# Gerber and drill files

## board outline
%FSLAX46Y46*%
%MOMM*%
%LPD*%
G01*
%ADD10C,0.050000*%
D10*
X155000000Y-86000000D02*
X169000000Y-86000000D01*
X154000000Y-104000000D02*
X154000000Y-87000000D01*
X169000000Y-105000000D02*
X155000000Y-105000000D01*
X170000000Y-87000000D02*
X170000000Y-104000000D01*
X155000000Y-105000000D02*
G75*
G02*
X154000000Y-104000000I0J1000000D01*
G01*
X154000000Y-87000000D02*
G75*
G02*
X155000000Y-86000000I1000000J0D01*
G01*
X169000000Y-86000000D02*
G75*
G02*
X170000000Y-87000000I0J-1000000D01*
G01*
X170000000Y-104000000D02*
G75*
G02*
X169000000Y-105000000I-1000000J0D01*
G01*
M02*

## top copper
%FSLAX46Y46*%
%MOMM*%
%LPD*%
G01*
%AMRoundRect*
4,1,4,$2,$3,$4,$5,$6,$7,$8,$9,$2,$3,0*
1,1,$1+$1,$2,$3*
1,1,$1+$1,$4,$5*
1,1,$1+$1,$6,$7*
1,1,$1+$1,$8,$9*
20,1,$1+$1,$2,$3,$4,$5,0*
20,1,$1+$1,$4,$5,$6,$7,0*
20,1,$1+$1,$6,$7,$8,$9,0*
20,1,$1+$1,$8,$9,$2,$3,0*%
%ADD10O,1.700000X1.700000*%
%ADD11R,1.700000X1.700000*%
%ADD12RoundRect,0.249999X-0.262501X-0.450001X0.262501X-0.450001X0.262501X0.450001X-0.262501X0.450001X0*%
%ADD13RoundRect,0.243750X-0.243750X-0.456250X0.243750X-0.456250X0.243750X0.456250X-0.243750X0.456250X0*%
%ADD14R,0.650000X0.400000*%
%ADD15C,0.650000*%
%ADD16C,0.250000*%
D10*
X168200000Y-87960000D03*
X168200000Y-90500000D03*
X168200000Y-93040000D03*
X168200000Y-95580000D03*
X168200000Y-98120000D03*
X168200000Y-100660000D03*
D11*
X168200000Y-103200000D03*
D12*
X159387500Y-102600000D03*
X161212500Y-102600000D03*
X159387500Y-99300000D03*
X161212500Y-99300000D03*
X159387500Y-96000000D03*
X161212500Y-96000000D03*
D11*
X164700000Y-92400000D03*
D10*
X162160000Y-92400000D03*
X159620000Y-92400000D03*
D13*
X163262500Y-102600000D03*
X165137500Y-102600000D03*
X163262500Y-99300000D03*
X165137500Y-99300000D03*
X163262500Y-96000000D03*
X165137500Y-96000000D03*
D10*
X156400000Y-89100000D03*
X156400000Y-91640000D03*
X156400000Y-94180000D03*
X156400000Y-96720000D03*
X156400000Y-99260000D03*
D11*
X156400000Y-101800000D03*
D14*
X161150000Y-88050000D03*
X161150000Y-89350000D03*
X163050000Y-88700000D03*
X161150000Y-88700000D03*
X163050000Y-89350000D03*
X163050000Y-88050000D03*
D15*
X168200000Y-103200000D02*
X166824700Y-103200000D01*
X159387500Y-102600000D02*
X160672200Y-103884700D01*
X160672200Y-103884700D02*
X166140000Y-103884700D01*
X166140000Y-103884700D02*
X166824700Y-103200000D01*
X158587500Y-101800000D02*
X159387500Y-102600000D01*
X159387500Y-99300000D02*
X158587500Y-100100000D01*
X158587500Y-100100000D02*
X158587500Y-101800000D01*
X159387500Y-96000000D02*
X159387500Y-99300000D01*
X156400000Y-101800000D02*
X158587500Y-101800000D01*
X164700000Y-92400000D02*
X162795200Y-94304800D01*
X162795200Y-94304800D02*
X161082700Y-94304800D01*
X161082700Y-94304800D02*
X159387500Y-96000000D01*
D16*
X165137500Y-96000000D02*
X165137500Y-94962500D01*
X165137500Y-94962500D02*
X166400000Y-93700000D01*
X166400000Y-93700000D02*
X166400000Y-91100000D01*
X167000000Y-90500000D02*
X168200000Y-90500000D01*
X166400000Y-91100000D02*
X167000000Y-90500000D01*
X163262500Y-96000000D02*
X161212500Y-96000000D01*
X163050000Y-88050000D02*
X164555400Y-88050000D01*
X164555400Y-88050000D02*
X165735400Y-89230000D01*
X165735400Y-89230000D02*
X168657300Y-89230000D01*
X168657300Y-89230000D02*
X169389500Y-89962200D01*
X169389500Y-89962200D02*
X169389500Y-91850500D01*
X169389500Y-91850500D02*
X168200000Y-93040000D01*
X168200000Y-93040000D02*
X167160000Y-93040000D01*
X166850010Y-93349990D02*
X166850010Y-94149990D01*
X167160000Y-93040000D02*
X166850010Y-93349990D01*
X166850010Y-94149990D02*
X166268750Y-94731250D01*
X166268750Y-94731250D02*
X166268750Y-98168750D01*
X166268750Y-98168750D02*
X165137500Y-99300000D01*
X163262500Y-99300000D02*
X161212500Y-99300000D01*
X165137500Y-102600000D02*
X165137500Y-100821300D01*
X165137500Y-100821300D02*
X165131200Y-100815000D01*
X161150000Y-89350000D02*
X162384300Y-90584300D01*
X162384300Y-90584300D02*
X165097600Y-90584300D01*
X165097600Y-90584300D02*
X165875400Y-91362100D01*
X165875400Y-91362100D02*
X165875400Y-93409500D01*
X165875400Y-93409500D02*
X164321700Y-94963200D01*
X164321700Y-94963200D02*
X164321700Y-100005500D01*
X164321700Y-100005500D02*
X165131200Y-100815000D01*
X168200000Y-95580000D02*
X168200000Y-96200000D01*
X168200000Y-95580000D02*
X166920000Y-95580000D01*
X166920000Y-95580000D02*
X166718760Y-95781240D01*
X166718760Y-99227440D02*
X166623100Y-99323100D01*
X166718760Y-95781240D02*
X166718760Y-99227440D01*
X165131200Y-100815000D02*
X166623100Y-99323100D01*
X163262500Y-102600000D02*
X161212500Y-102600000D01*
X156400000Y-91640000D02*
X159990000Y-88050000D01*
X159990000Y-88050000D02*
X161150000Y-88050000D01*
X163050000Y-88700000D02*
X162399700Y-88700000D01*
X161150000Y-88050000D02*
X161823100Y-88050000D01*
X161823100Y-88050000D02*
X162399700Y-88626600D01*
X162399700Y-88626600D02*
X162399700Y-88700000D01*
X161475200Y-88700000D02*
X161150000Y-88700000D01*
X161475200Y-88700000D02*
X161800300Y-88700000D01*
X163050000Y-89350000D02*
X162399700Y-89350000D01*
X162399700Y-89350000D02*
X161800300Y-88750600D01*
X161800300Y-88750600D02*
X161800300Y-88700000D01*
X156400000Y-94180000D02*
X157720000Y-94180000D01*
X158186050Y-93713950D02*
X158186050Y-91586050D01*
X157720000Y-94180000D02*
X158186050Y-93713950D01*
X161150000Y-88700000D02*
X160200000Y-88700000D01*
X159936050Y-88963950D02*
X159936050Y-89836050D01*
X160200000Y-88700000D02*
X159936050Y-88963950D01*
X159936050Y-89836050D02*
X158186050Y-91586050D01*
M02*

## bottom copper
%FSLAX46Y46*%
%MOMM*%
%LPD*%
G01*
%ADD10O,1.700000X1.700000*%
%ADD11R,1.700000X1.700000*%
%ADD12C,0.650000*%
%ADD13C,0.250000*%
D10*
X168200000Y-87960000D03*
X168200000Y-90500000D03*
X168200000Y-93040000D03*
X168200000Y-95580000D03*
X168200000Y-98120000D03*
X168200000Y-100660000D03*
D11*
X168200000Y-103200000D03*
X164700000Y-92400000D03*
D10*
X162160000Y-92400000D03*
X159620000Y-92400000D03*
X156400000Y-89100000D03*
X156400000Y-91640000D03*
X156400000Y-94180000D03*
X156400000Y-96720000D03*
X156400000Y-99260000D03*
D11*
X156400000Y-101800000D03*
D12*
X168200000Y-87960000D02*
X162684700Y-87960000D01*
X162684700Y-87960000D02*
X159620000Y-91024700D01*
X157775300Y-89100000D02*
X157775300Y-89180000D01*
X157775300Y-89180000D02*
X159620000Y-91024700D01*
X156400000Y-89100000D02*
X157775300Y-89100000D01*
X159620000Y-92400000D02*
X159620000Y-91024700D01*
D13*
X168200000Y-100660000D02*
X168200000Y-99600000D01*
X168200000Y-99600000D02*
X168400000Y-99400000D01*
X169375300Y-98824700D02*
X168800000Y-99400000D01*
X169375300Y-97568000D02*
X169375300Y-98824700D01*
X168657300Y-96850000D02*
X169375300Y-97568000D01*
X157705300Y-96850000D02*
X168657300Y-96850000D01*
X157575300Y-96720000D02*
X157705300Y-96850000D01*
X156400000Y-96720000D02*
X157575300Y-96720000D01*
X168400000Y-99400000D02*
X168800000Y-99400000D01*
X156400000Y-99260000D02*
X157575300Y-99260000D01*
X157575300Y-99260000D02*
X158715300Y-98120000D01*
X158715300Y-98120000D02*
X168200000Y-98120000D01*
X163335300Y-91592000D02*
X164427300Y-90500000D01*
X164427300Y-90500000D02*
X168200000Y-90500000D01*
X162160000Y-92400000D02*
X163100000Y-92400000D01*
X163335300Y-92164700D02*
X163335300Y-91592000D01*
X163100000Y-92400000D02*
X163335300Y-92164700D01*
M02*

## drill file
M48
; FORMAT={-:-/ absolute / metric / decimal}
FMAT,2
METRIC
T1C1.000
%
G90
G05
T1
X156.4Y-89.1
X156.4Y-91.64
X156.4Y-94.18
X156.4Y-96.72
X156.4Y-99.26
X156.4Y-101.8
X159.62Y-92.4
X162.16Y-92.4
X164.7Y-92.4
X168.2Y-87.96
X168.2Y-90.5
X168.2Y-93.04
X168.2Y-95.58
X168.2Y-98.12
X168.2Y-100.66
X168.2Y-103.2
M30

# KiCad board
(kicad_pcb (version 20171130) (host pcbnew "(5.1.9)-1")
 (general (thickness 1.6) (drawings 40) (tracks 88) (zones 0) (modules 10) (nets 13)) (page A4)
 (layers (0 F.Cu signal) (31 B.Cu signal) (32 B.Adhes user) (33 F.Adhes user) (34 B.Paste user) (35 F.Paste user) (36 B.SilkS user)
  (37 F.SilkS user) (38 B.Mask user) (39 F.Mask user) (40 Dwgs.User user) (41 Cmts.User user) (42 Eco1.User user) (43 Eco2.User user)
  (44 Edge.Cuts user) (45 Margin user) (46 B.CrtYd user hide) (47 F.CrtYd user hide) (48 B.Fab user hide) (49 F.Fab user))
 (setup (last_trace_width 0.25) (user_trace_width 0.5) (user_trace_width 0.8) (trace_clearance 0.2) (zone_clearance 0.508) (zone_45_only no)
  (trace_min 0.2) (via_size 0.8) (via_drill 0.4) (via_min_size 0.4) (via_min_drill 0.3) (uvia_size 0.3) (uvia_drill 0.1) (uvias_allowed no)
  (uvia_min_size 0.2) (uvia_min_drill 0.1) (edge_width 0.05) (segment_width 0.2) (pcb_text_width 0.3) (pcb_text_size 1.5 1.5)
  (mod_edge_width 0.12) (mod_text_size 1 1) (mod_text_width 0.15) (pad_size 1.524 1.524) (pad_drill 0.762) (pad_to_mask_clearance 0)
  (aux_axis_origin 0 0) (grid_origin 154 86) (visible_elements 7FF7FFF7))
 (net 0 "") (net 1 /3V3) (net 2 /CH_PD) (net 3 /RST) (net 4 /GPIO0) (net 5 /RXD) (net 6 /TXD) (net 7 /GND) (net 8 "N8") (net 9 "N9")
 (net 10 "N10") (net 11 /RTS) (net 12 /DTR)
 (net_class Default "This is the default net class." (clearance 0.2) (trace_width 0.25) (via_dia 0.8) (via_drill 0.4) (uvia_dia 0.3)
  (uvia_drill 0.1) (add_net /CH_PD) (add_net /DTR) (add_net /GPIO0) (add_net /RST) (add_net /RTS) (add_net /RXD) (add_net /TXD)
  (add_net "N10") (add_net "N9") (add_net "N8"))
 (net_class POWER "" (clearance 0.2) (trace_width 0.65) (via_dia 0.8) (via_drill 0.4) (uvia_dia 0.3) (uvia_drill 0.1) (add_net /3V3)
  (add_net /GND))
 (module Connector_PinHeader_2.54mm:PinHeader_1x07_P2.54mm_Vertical (layer F.Cu) (at 168.2 103.2 180)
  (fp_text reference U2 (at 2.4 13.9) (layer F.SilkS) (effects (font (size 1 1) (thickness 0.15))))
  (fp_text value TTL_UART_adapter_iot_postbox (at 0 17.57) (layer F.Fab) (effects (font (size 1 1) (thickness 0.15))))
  (pad 7 thru_hole oval (at 0 15.24 180) (size 1.7 1.7) (drill 1) (layers *.Cu *.Mask) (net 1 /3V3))
  (pad 6 thru_hole oval (at 0 12.7 180) (size 1.7 1.7) (drill 1) (layers *.Cu *.Mask) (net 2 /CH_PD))
  (pad 5 thru_hole oval (at 0 10.16 180) (size 1.7 1.7) (drill 1) (layers *.Cu *.Mask) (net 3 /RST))
  (pad 4 thru_hole oval (at 0 7.62 180) (size 1.7 1.7) (drill 1) (layers *.Cu *.Mask) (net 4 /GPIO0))
  (pad 3 thru_hole oval (at 0 5.08 180) (size 1.7 1.7) (drill 1) (layers *.Cu *.Mask) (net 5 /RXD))
  (pad 2 thru_hole oval (at 0 2.54 180) (size 1.7 1.7) (drill 1) (layers *.Cu *.Mask) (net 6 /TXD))
  (pad 1 thru_hole rect (at 0 0 180) (size 1.7 1.7) (drill 1) (layers *.Cu *.Mask) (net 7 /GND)))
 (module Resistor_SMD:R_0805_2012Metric (layer F.Cu) (at 160.3 102.6)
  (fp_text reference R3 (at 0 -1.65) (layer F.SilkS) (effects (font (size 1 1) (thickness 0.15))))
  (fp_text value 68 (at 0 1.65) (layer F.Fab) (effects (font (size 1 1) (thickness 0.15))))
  (pad 1 smd roundrect (at -0.9125 0) (size 1.025 1.4) (layers F.Cu F.Paste F.Mask) (roundrect_rratio 0.2439014634146341) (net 7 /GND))
  (pad 2 smd roundrect (at 0.9125 0) (size 1.025 1.4) (layers F.Cu F.Paste F.Mask) (roundrect_rratio 0.2439014634146341) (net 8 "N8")))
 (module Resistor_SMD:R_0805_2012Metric (layer F.Cu) (at 160.3 99.3)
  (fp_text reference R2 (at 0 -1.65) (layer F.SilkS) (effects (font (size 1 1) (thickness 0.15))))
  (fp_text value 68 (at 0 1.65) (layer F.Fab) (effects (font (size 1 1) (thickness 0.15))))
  (pad 1 smd roundrect (at -0.9125 0) (size 1.025 1.4) (layers F.Cu F.Paste F.Mask) (roundrect_rratio 0.2439014634146341) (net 7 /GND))
  (pad 2 smd roundrect (at 0.9125 0) (size 1.025 1.4) (layers F.Cu F.Paste F.Mask) (roundrect_rratio 0.2439014634146341) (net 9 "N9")))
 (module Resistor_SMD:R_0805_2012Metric (layer F.Cu) (at 160.3 96)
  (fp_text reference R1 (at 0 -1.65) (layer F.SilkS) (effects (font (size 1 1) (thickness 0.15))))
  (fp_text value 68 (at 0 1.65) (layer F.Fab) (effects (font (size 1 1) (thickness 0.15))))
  (pad 1 smd roundrect (at -0.9125 0) (size 1.025 1.4) (layers F.Cu F.Paste F.Mask) (roundrect_rratio 0.2439014634146341) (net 7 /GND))
  (pad 2 smd roundrect (at 0.9125 0) (size 1.025 1.4) (layers F.Cu F.Paste F.Mask) (roundrect_rratio 0.2439014634146341) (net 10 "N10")))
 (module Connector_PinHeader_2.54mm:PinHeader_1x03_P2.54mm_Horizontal (layer B.Cu) (at 164.7 92.4 90)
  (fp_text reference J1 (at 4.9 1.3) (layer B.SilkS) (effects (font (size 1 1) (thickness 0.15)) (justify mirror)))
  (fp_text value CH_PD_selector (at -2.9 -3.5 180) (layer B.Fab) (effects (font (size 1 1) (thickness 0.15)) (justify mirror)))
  (pad 1 thru_hole rect (at 0 0 90) (size 1.7 1.7) (drill 1) (layers *.Cu *.Mask) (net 7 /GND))
  (pad 2 thru_hole oval (at 0 -2.54 90) (size 1.7 1.7) (drill 1) (layers *.Cu *.Mask) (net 2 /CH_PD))
  (pad 3 thru_hole oval (at 0 -5.08 90) (size 1.7 1.7) (drill 1) (layers *.Cu *.Mask) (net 1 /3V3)))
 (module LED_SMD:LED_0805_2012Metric (layer F.Cu) (at 164.2 102.6)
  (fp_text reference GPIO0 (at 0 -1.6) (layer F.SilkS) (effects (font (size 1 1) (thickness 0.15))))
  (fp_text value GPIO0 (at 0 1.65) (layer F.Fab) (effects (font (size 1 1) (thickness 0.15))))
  (pad 1 smd roundrect (at -0.9375 0) (size 0.975 1.4) (layers F.Cu F.Paste F.Mask) (roundrect_rratio 0.25) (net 8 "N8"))
  (pad 2 smd roundrect (at 0.9375 0) (size 0.975 1.4) (layers F.Cu F.Paste F.Mask) (roundrect_rratio 0.25) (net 4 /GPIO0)))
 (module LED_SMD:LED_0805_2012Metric (layer F.Cu) (at 164.2 99.3)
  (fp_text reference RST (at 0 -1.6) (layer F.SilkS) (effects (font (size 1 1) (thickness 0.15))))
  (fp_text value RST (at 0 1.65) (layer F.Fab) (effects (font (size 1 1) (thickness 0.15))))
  (pad 1 smd roundrect (at -0.9375 0) (size 0.975 1.4) (layers F.Cu F.Paste F.Mask) (roundrect_rratio 0.25) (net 9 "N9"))
  (pad 2 smd roundrect (at 0.9375 0) (size 0.975 1.4) (layers F.Cu F.Paste F.Mask) (roundrect_rratio 0.25) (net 3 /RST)))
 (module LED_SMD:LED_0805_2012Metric (layer F.Cu) (at 164.2 96)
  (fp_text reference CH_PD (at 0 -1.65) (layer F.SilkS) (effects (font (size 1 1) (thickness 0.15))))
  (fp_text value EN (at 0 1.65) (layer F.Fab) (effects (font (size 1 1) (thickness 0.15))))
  (pad 1 smd roundrect (at -0.9375 0) (size 0.975 1.4) (layers F.Cu F.Paste F.Mask) (roundrect_rratio 0.25) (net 10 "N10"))
  (pad 2 smd roundrect (at 0.9375 0) (size 0.975 1.4) (layers F.Cu F.Paste F.Mask) (roundrect_rratio 0.25) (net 2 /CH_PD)))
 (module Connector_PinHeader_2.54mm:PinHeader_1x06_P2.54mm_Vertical (layer F.Cu) (at 156.4 101.8 180)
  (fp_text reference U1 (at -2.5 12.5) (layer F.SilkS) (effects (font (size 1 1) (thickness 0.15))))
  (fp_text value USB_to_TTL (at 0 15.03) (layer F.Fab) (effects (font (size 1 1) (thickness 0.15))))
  (pad 6 thru_hole oval (at 0 12.7 180) (size 1.7 1.7) (drill 1) (layers *.Cu *.Mask) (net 1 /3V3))
  (pad 5 thru_hole oval (at 0 10.16 180) (size 1.7 1.7) (drill 1) (layers *.Cu *.Mask) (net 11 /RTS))
  (pad 4 thru_hole oval (at 0 7.62 180) (size 1.7 1.7) (drill 1) (layers *.Cu *.Mask) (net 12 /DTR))
  (pad 3 thru_hole oval (at 0 5.08 180) (size 1.7 1.7) (drill 1) (layers *.Cu *.Mask) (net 6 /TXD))
  (pad 2 thru_hole oval (at 0 2.54 180) (size 1.7 1.7) (drill 1) (layers *.Cu *.Mask) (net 5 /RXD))
  (pad 1 thru_hole rect (at 0 0 180) (size 1.7 1.7) (drill 1) (layers *.Cu *.Mask) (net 7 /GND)))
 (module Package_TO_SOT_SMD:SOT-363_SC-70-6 (layer F.Cu) (at 162.1 88.7)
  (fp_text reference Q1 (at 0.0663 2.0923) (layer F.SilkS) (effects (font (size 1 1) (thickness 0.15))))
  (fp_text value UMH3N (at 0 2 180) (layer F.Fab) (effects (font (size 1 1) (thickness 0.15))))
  (pad 1 smd rect (at -0.95 -0.65) (size 0.65 0.4) (layers F.Cu F.Paste F.Mask) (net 11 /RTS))
  (pad 3 smd rect (at -0.95 0.65) (size 0.65 0.4) (layers F.Cu F.Paste F.Mask) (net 4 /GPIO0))
  (pad 5 smd rect (at 0.95 0) (size 0.65 0.4) (layers F.Cu F.Paste F.Mask) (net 11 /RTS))
  (pad 2 smd rect (at -0.95 0) (size 0.65 0.4) (layers F.Cu F.Paste F.Mask) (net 12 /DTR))
  (pad 4 smd rect (at 0.95 0.65) (size 0.65 0.4) (layers F.Cu F.Paste F.Mask) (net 12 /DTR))
  (pad 6 smd rect (at 0.95 -0.65) (size 0.65 0.4) (layers F.Cu F.Paste F.Mask) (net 3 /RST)))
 (gr_line (start 155 86) (end 169 86) (layer Edge.Cuts) (width 0.05))
 (gr_line (start 154 104) (end 154 87) (layer Edge.Cuts) (width 0.05))
 (gr_line (start 169 105) (end 155 105) (layer Edge.Cuts) (width 0.05))
 (gr_line (start 170 87) (end 170 104) (layer Edge.Cuts) (width 0.05))
 (gr_arc (start 155 104) (end 154 104) (angle -90) (layer Edge.Cuts) (width 0.05))
 (gr_arc (start 155 87) (end 155 86) (angle -90) (layer Edge.Cuts) (width 0.05))
 (gr_arc (start 169 87) (end 170 87) (angle -90) (layer Edge.Cuts) (width 0.05))
 (gr_arc (start 169 104) (end 169 105) (angle -90) (layer Edge.Cuts) (width 0.05))
 (segment (start 168.2 87.96) (end 162.6847 87.96) (width 0.65) (layer B.Cu) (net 1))
 (segment (start 162.6847 87.96) (end 159.62 91.0247) (width 0.65) (layer B.Cu) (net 1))
 (segment (start 157.7753 89.1) (end 157.7753 89.18) (width 0.65) (layer B.Cu) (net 1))
 (segment (start 157.7753 89.18) (end 159.62 91.0247) (width 0.65) (layer B.Cu) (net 1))
 (segment (start 156.4 89.1) (end 157.7753 89.1) (width 0.65) (layer B.Cu) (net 1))
 (segment (start 159.62 92.4) (end 159.62 91.0247) (width 0.65) (layer B.Cu) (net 1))
 (segment (start 168.2 100.66) (end 168.2 99.6) (width 0.25) (layer B.Cu) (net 6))
 (segment (start 168.2 99.6) (end 168.4 99.4) (width 0.25) (layer B.Cu) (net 6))
 (segment (start 169.3753 98.8247) (end 168.8 99.4) (width 0.25) (layer B.Cu) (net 6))
 (segment (start 169.3753 97.568) (end 169.3753 98.8247) (width 0.25) (layer B.Cu) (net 6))
 (segment (start 168.6573 96.85) (end 169.3753 97.568) (width 0.25) (layer B.Cu) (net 6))
 (segment (start 157.7053 96.85) (end 168.6573 96.85) (width 0.25) (layer B.Cu) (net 6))
 (segment (start 157.5753 96.72) (end 157.7053 96.85) (width 0.25) (layer B.Cu) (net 6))
 (segment (start 156.4 96.72) (end 157.5753 96.72) (width 0.25) (layer B.Cu) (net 6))
 (segment (start 168.4 99.4) (end 168.8 99.4) (width 0.25) (layer B.Cu) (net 6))
 (segment (start 156.4 99.26) (end 157.5753 99.26) (width 0.25) (layer B.Cu) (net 5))
 (segment (start 157.5753 99.26) (end 158.7153 98.12) (width 0.25) (layer B.Cu) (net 5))
 (segment (start 158.7153 98.12) (end 168.2 98.12) (width 0.25) (layer B.Cu) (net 5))
 (segment (start 168.2 103.2) (end 166.8247 103.2) (width 0.65) (layer F.Cu) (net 7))
 (segment (start 159.3875 102.6) (end 160.6722 103.8847) (width 0.65) (layer F.Cu) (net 7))
 (segment (start 160.6722 103.8847) (end 166.14 103.8847) (width 0.65) (layer F.Cu) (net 7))
 (segment (start 166.14 103.8847) (end 166.8247 103.2) (width 0.65) (layer F.Cu) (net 7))
 (segment (start 158.5875 101.8) (end 159.3875 102.6) (width 0.65) (layer F.Cu) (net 7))
 (segment (start 159.3875 99.3) (end 158.5875 100.1) (width 0.65) (layer F.Cu) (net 7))
 (segment (start 158.5875 100.1) (end 158.5875 101.8) (width 0.65) (layer F.Cu) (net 7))
 (segment (start 159.3875 96) (end 159.3875 99.3) (width 0.65) (layer F.Cu) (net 7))
 (segment (start 156.4 101.8) (end 158.5875 101.8) (width 0.65) (layer F.Cu) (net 7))
 (segment (start 164.7 92.4) (end 162.7952 94.3048) (width 0.65) (layer F.Cu) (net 7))
 (segment (start 162.7952 94.3048) (end 161.0827 94.3048) (width 0.65) (layer F.Cu) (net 7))
 (segment (start 161.0827 94.3048) (end 159.3875 96) (width 0.65) (layer F.Cu) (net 7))
 (segment (start 163.3353 91.592) (end 164.4273 90.5) (width 0.25) (layer B.Cu) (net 2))
 (segment (start 164.4273 90.5) (end 168.2 90.5) (width 0.25) (layer B.Cu) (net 2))
 (segment (start 165.1375 96) (end 165.1375 94.9625) (width 0.25) (layer F.Cu) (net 2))
 (segment (start 165.1375 94.9625) (end 166.4 93.7) (width 0.25) (layer F.Cu) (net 2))
 (segment (start 166.4 93.7) (end 166.4 91.1) (width 0.25) (layer F.Cu) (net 2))
 (segment (start 167 90.5) (end 168.2 90.5) (width 0.25) (layer F.Cu) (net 2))
 (segment (start 166.4 91.1) (end 167 90.5) (width 0.25) (layer F.Cu) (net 2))
 (segment (start 162.16 92.4) (end 163.1 92.4) (width 0.25) (layer B.Cu) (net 2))
 (segment (start 163.3353 92.1647) (end 163.3353 91.592) (width 0.25) (layer B.Cu) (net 2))
 (segment (start 163.1 92.4) (end 163.3353 92.1647) (width 0.25) (layer B.Cu) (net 2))
 (segment (start 163.2625 96) (end 161.2125 96) (width 0.25) (layer F.Cu) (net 10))
 (segment (start 163.05 88.05) (end 164.5554 88.05) (width 0.25) (layer F.Cu) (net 3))
 (segment (start 164.5554 88.05) (end 165.7354 89.23) (width 0.25) (layer F.Cu) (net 3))
 (segment (start 165.7354 89.23) (end 168.6573 89.23) (width 0.25) (layer F.Cu) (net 3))
 (segment (start 168.6573 89.23) (end 169.3895 89.9622) (width 0.25) (layer F.Cu) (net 3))
 (segment (start 169.3895 89.9622) (end 169.3895 91.8505) (width 0.25) (layer F.Cu) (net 3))
 (segment (start 169.3895 91.8505) (end 168.2 93.04) (width 0.25) (layer F.Cu) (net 3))
 (segment (start 168.2 93.04) (end 167.16 93.04) (width 0.25) (layer F.Cu) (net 3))
 (segment (start 166.85001 93.34999) (end 166.85001 94.14999) (width 0.25) (layer F.Cu) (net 3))
 (segment (start 167.16 93.04) (end 166.85001 93.34999) (width 0.25) (layer F.Cu) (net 3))
 (segment (start 166.85001 94.14999) (end 166.26875 94.73125) (width 0.25) (layer F.Cu) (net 3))
 (segment (start 166.26875 94.73125) (end 166.26875 98.16875) (width 0.25) (layer F.Cu) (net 3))
 (segment (start 166.26875 98.16875) (end 165.1375 99.3) (width 0.25) (layer F.Cu) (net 3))
 (segment (start 163.2625 99.3) (end 161.2125 99.3) (width 0.25) (layer F.Cu) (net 9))
 (segment (start 165.1375 102.6) (end 165.1375 100.8213) (width 0.25) (layer F.Cu) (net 4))
 (segment (start 165.1375 100.8213) (end 165.1312 100.815) (width 0.25) (layer F.Cu) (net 4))
 (segment (start 161.15 89.35) (end 162.3843 90.5843) (width 0.25) (layer F.Cu) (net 4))
 (segment (start 162.3843 90.5843) (end 165.0976 90.5843) (width 0.25) (layer F.Cu) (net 4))
 (segment (start 165.0976 90.5843) (end 165.8754 91.3621) (width 0.25) (layer F.Cu) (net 4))
 (segment (start 165.8754 91.3621) (end 165.8754 93.4095) (width 0.25) (layer F.Cu) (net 4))
 (segment (start 165.8754 93.4095) (end 164.3217 94.9632) (width 0.25) (layer F.Cu) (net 4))
 (segment (start 164.3217 94.9632) (end 164.3217 100.0055) (width 0.25) (layer F.Cu) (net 4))
 (segment (start 164.3217 100.0055) (end 165.1312 100.815) (width 0.25) (layer F.Cu) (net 4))
 (segment (start 168.2 95.58) (end 168.2 96.2) (width 0.25) (layer F.Cu) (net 4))
 (segment (start 168.2 95.58) (end 166.92 95.58) (width 0.25) (layer F.Cu) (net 4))
 (segment (start 166.92 95.58) (end 166.71876 95.78124) (width 0.25) (layer F.Cu) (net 4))
 (segment (start 166.71876 99.22744) (end 166.6231 99.3231) (width 0.25) (layer F.Cu) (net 4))
 (segment (start 166.71876 95.78124) (end 166.71876 99.22744) (width 0.25) (layer F.Cu) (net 4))
 (segment (start 165.1312 100.815) (end 166.6231 99.3231) (width 0.25) (layer F.Cu) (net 4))
 (segment (start 163.2625 102.6) (end 161.2125 102.6) (width 0.25) (layer F.Cu) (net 8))
 (segment (start 156.4 91.64) (end 159.99 88.05) (width 0.25) (layer F.Cu) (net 11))
 (segment (start 159.99 88.05) (end 161.15 88.05) (width 0.25) (layer F.Cu) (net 11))
 (segment (start 163.05 88.7) (end 162.3997 88.7) (width 0.25) (layer F.Cu) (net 11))
 (segment (start 161.15 88.05) (end 161.8231 88.05) (width 0.25) (layer F.Cu) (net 11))
 (segment (start 161.8231 88.05) (end 162.3997 88.6266) (width 0.25) (layer F.Cu) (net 11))
 (segment (start 162.3997 88.6266) (end 162.3997 88.7) (width 0.25) (layer F.Cu) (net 11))
 (segment (start 161.4752 88.7) (end 161.15 88.7) (width 0.25) (layer F.Cu) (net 12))
 (segment (start 161.4752 88.7) (end 161.8003 88.7) (width 0.25) (layer F.Cu) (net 12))
 (segment (start 163.05 89.35) (end 162.3997 89.35) (width 0.25) (layer F.Cu) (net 12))
 (segment (start 162.3997 89.35) (end 161.8003 88.7506) (width 0.25) (layer F.Cu) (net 12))
 (segment (start 161.8003 88.7506) (end 161.8003 88.7) (width 0.25) (layer F.Cu) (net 12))
 (segment (start 156.4 94.18) (end 157.72 94.18) (width 0.25) (layer F.Cu) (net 12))
 (segment (start 158.18605 93.71395) (end 158.18605 91.58605) (width 0.25) (layer F.Cu) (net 12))
 (segment (start 157.72 94.18) (end 158.18605 93.71395) (width 0.25) (layer F.Cu) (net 12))
 (segment (start 161.15 88.7) (end 160.2 88.7) (width 0.25) (layer F.Cu) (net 12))
 (segment (start 159.93605 88.96395) (end 159.93605 89.83605) (width 0.25) (layer F.Cu) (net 12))
 (segment (start 160.2 88.7) (end 159.93605 88.96395) (width 0.25) (layer F.Cu) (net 12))
 (segment (start 159.93605 89.83605) (end 158.18605 91.58605) (width 0.25) (layer F.Cu) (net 12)))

